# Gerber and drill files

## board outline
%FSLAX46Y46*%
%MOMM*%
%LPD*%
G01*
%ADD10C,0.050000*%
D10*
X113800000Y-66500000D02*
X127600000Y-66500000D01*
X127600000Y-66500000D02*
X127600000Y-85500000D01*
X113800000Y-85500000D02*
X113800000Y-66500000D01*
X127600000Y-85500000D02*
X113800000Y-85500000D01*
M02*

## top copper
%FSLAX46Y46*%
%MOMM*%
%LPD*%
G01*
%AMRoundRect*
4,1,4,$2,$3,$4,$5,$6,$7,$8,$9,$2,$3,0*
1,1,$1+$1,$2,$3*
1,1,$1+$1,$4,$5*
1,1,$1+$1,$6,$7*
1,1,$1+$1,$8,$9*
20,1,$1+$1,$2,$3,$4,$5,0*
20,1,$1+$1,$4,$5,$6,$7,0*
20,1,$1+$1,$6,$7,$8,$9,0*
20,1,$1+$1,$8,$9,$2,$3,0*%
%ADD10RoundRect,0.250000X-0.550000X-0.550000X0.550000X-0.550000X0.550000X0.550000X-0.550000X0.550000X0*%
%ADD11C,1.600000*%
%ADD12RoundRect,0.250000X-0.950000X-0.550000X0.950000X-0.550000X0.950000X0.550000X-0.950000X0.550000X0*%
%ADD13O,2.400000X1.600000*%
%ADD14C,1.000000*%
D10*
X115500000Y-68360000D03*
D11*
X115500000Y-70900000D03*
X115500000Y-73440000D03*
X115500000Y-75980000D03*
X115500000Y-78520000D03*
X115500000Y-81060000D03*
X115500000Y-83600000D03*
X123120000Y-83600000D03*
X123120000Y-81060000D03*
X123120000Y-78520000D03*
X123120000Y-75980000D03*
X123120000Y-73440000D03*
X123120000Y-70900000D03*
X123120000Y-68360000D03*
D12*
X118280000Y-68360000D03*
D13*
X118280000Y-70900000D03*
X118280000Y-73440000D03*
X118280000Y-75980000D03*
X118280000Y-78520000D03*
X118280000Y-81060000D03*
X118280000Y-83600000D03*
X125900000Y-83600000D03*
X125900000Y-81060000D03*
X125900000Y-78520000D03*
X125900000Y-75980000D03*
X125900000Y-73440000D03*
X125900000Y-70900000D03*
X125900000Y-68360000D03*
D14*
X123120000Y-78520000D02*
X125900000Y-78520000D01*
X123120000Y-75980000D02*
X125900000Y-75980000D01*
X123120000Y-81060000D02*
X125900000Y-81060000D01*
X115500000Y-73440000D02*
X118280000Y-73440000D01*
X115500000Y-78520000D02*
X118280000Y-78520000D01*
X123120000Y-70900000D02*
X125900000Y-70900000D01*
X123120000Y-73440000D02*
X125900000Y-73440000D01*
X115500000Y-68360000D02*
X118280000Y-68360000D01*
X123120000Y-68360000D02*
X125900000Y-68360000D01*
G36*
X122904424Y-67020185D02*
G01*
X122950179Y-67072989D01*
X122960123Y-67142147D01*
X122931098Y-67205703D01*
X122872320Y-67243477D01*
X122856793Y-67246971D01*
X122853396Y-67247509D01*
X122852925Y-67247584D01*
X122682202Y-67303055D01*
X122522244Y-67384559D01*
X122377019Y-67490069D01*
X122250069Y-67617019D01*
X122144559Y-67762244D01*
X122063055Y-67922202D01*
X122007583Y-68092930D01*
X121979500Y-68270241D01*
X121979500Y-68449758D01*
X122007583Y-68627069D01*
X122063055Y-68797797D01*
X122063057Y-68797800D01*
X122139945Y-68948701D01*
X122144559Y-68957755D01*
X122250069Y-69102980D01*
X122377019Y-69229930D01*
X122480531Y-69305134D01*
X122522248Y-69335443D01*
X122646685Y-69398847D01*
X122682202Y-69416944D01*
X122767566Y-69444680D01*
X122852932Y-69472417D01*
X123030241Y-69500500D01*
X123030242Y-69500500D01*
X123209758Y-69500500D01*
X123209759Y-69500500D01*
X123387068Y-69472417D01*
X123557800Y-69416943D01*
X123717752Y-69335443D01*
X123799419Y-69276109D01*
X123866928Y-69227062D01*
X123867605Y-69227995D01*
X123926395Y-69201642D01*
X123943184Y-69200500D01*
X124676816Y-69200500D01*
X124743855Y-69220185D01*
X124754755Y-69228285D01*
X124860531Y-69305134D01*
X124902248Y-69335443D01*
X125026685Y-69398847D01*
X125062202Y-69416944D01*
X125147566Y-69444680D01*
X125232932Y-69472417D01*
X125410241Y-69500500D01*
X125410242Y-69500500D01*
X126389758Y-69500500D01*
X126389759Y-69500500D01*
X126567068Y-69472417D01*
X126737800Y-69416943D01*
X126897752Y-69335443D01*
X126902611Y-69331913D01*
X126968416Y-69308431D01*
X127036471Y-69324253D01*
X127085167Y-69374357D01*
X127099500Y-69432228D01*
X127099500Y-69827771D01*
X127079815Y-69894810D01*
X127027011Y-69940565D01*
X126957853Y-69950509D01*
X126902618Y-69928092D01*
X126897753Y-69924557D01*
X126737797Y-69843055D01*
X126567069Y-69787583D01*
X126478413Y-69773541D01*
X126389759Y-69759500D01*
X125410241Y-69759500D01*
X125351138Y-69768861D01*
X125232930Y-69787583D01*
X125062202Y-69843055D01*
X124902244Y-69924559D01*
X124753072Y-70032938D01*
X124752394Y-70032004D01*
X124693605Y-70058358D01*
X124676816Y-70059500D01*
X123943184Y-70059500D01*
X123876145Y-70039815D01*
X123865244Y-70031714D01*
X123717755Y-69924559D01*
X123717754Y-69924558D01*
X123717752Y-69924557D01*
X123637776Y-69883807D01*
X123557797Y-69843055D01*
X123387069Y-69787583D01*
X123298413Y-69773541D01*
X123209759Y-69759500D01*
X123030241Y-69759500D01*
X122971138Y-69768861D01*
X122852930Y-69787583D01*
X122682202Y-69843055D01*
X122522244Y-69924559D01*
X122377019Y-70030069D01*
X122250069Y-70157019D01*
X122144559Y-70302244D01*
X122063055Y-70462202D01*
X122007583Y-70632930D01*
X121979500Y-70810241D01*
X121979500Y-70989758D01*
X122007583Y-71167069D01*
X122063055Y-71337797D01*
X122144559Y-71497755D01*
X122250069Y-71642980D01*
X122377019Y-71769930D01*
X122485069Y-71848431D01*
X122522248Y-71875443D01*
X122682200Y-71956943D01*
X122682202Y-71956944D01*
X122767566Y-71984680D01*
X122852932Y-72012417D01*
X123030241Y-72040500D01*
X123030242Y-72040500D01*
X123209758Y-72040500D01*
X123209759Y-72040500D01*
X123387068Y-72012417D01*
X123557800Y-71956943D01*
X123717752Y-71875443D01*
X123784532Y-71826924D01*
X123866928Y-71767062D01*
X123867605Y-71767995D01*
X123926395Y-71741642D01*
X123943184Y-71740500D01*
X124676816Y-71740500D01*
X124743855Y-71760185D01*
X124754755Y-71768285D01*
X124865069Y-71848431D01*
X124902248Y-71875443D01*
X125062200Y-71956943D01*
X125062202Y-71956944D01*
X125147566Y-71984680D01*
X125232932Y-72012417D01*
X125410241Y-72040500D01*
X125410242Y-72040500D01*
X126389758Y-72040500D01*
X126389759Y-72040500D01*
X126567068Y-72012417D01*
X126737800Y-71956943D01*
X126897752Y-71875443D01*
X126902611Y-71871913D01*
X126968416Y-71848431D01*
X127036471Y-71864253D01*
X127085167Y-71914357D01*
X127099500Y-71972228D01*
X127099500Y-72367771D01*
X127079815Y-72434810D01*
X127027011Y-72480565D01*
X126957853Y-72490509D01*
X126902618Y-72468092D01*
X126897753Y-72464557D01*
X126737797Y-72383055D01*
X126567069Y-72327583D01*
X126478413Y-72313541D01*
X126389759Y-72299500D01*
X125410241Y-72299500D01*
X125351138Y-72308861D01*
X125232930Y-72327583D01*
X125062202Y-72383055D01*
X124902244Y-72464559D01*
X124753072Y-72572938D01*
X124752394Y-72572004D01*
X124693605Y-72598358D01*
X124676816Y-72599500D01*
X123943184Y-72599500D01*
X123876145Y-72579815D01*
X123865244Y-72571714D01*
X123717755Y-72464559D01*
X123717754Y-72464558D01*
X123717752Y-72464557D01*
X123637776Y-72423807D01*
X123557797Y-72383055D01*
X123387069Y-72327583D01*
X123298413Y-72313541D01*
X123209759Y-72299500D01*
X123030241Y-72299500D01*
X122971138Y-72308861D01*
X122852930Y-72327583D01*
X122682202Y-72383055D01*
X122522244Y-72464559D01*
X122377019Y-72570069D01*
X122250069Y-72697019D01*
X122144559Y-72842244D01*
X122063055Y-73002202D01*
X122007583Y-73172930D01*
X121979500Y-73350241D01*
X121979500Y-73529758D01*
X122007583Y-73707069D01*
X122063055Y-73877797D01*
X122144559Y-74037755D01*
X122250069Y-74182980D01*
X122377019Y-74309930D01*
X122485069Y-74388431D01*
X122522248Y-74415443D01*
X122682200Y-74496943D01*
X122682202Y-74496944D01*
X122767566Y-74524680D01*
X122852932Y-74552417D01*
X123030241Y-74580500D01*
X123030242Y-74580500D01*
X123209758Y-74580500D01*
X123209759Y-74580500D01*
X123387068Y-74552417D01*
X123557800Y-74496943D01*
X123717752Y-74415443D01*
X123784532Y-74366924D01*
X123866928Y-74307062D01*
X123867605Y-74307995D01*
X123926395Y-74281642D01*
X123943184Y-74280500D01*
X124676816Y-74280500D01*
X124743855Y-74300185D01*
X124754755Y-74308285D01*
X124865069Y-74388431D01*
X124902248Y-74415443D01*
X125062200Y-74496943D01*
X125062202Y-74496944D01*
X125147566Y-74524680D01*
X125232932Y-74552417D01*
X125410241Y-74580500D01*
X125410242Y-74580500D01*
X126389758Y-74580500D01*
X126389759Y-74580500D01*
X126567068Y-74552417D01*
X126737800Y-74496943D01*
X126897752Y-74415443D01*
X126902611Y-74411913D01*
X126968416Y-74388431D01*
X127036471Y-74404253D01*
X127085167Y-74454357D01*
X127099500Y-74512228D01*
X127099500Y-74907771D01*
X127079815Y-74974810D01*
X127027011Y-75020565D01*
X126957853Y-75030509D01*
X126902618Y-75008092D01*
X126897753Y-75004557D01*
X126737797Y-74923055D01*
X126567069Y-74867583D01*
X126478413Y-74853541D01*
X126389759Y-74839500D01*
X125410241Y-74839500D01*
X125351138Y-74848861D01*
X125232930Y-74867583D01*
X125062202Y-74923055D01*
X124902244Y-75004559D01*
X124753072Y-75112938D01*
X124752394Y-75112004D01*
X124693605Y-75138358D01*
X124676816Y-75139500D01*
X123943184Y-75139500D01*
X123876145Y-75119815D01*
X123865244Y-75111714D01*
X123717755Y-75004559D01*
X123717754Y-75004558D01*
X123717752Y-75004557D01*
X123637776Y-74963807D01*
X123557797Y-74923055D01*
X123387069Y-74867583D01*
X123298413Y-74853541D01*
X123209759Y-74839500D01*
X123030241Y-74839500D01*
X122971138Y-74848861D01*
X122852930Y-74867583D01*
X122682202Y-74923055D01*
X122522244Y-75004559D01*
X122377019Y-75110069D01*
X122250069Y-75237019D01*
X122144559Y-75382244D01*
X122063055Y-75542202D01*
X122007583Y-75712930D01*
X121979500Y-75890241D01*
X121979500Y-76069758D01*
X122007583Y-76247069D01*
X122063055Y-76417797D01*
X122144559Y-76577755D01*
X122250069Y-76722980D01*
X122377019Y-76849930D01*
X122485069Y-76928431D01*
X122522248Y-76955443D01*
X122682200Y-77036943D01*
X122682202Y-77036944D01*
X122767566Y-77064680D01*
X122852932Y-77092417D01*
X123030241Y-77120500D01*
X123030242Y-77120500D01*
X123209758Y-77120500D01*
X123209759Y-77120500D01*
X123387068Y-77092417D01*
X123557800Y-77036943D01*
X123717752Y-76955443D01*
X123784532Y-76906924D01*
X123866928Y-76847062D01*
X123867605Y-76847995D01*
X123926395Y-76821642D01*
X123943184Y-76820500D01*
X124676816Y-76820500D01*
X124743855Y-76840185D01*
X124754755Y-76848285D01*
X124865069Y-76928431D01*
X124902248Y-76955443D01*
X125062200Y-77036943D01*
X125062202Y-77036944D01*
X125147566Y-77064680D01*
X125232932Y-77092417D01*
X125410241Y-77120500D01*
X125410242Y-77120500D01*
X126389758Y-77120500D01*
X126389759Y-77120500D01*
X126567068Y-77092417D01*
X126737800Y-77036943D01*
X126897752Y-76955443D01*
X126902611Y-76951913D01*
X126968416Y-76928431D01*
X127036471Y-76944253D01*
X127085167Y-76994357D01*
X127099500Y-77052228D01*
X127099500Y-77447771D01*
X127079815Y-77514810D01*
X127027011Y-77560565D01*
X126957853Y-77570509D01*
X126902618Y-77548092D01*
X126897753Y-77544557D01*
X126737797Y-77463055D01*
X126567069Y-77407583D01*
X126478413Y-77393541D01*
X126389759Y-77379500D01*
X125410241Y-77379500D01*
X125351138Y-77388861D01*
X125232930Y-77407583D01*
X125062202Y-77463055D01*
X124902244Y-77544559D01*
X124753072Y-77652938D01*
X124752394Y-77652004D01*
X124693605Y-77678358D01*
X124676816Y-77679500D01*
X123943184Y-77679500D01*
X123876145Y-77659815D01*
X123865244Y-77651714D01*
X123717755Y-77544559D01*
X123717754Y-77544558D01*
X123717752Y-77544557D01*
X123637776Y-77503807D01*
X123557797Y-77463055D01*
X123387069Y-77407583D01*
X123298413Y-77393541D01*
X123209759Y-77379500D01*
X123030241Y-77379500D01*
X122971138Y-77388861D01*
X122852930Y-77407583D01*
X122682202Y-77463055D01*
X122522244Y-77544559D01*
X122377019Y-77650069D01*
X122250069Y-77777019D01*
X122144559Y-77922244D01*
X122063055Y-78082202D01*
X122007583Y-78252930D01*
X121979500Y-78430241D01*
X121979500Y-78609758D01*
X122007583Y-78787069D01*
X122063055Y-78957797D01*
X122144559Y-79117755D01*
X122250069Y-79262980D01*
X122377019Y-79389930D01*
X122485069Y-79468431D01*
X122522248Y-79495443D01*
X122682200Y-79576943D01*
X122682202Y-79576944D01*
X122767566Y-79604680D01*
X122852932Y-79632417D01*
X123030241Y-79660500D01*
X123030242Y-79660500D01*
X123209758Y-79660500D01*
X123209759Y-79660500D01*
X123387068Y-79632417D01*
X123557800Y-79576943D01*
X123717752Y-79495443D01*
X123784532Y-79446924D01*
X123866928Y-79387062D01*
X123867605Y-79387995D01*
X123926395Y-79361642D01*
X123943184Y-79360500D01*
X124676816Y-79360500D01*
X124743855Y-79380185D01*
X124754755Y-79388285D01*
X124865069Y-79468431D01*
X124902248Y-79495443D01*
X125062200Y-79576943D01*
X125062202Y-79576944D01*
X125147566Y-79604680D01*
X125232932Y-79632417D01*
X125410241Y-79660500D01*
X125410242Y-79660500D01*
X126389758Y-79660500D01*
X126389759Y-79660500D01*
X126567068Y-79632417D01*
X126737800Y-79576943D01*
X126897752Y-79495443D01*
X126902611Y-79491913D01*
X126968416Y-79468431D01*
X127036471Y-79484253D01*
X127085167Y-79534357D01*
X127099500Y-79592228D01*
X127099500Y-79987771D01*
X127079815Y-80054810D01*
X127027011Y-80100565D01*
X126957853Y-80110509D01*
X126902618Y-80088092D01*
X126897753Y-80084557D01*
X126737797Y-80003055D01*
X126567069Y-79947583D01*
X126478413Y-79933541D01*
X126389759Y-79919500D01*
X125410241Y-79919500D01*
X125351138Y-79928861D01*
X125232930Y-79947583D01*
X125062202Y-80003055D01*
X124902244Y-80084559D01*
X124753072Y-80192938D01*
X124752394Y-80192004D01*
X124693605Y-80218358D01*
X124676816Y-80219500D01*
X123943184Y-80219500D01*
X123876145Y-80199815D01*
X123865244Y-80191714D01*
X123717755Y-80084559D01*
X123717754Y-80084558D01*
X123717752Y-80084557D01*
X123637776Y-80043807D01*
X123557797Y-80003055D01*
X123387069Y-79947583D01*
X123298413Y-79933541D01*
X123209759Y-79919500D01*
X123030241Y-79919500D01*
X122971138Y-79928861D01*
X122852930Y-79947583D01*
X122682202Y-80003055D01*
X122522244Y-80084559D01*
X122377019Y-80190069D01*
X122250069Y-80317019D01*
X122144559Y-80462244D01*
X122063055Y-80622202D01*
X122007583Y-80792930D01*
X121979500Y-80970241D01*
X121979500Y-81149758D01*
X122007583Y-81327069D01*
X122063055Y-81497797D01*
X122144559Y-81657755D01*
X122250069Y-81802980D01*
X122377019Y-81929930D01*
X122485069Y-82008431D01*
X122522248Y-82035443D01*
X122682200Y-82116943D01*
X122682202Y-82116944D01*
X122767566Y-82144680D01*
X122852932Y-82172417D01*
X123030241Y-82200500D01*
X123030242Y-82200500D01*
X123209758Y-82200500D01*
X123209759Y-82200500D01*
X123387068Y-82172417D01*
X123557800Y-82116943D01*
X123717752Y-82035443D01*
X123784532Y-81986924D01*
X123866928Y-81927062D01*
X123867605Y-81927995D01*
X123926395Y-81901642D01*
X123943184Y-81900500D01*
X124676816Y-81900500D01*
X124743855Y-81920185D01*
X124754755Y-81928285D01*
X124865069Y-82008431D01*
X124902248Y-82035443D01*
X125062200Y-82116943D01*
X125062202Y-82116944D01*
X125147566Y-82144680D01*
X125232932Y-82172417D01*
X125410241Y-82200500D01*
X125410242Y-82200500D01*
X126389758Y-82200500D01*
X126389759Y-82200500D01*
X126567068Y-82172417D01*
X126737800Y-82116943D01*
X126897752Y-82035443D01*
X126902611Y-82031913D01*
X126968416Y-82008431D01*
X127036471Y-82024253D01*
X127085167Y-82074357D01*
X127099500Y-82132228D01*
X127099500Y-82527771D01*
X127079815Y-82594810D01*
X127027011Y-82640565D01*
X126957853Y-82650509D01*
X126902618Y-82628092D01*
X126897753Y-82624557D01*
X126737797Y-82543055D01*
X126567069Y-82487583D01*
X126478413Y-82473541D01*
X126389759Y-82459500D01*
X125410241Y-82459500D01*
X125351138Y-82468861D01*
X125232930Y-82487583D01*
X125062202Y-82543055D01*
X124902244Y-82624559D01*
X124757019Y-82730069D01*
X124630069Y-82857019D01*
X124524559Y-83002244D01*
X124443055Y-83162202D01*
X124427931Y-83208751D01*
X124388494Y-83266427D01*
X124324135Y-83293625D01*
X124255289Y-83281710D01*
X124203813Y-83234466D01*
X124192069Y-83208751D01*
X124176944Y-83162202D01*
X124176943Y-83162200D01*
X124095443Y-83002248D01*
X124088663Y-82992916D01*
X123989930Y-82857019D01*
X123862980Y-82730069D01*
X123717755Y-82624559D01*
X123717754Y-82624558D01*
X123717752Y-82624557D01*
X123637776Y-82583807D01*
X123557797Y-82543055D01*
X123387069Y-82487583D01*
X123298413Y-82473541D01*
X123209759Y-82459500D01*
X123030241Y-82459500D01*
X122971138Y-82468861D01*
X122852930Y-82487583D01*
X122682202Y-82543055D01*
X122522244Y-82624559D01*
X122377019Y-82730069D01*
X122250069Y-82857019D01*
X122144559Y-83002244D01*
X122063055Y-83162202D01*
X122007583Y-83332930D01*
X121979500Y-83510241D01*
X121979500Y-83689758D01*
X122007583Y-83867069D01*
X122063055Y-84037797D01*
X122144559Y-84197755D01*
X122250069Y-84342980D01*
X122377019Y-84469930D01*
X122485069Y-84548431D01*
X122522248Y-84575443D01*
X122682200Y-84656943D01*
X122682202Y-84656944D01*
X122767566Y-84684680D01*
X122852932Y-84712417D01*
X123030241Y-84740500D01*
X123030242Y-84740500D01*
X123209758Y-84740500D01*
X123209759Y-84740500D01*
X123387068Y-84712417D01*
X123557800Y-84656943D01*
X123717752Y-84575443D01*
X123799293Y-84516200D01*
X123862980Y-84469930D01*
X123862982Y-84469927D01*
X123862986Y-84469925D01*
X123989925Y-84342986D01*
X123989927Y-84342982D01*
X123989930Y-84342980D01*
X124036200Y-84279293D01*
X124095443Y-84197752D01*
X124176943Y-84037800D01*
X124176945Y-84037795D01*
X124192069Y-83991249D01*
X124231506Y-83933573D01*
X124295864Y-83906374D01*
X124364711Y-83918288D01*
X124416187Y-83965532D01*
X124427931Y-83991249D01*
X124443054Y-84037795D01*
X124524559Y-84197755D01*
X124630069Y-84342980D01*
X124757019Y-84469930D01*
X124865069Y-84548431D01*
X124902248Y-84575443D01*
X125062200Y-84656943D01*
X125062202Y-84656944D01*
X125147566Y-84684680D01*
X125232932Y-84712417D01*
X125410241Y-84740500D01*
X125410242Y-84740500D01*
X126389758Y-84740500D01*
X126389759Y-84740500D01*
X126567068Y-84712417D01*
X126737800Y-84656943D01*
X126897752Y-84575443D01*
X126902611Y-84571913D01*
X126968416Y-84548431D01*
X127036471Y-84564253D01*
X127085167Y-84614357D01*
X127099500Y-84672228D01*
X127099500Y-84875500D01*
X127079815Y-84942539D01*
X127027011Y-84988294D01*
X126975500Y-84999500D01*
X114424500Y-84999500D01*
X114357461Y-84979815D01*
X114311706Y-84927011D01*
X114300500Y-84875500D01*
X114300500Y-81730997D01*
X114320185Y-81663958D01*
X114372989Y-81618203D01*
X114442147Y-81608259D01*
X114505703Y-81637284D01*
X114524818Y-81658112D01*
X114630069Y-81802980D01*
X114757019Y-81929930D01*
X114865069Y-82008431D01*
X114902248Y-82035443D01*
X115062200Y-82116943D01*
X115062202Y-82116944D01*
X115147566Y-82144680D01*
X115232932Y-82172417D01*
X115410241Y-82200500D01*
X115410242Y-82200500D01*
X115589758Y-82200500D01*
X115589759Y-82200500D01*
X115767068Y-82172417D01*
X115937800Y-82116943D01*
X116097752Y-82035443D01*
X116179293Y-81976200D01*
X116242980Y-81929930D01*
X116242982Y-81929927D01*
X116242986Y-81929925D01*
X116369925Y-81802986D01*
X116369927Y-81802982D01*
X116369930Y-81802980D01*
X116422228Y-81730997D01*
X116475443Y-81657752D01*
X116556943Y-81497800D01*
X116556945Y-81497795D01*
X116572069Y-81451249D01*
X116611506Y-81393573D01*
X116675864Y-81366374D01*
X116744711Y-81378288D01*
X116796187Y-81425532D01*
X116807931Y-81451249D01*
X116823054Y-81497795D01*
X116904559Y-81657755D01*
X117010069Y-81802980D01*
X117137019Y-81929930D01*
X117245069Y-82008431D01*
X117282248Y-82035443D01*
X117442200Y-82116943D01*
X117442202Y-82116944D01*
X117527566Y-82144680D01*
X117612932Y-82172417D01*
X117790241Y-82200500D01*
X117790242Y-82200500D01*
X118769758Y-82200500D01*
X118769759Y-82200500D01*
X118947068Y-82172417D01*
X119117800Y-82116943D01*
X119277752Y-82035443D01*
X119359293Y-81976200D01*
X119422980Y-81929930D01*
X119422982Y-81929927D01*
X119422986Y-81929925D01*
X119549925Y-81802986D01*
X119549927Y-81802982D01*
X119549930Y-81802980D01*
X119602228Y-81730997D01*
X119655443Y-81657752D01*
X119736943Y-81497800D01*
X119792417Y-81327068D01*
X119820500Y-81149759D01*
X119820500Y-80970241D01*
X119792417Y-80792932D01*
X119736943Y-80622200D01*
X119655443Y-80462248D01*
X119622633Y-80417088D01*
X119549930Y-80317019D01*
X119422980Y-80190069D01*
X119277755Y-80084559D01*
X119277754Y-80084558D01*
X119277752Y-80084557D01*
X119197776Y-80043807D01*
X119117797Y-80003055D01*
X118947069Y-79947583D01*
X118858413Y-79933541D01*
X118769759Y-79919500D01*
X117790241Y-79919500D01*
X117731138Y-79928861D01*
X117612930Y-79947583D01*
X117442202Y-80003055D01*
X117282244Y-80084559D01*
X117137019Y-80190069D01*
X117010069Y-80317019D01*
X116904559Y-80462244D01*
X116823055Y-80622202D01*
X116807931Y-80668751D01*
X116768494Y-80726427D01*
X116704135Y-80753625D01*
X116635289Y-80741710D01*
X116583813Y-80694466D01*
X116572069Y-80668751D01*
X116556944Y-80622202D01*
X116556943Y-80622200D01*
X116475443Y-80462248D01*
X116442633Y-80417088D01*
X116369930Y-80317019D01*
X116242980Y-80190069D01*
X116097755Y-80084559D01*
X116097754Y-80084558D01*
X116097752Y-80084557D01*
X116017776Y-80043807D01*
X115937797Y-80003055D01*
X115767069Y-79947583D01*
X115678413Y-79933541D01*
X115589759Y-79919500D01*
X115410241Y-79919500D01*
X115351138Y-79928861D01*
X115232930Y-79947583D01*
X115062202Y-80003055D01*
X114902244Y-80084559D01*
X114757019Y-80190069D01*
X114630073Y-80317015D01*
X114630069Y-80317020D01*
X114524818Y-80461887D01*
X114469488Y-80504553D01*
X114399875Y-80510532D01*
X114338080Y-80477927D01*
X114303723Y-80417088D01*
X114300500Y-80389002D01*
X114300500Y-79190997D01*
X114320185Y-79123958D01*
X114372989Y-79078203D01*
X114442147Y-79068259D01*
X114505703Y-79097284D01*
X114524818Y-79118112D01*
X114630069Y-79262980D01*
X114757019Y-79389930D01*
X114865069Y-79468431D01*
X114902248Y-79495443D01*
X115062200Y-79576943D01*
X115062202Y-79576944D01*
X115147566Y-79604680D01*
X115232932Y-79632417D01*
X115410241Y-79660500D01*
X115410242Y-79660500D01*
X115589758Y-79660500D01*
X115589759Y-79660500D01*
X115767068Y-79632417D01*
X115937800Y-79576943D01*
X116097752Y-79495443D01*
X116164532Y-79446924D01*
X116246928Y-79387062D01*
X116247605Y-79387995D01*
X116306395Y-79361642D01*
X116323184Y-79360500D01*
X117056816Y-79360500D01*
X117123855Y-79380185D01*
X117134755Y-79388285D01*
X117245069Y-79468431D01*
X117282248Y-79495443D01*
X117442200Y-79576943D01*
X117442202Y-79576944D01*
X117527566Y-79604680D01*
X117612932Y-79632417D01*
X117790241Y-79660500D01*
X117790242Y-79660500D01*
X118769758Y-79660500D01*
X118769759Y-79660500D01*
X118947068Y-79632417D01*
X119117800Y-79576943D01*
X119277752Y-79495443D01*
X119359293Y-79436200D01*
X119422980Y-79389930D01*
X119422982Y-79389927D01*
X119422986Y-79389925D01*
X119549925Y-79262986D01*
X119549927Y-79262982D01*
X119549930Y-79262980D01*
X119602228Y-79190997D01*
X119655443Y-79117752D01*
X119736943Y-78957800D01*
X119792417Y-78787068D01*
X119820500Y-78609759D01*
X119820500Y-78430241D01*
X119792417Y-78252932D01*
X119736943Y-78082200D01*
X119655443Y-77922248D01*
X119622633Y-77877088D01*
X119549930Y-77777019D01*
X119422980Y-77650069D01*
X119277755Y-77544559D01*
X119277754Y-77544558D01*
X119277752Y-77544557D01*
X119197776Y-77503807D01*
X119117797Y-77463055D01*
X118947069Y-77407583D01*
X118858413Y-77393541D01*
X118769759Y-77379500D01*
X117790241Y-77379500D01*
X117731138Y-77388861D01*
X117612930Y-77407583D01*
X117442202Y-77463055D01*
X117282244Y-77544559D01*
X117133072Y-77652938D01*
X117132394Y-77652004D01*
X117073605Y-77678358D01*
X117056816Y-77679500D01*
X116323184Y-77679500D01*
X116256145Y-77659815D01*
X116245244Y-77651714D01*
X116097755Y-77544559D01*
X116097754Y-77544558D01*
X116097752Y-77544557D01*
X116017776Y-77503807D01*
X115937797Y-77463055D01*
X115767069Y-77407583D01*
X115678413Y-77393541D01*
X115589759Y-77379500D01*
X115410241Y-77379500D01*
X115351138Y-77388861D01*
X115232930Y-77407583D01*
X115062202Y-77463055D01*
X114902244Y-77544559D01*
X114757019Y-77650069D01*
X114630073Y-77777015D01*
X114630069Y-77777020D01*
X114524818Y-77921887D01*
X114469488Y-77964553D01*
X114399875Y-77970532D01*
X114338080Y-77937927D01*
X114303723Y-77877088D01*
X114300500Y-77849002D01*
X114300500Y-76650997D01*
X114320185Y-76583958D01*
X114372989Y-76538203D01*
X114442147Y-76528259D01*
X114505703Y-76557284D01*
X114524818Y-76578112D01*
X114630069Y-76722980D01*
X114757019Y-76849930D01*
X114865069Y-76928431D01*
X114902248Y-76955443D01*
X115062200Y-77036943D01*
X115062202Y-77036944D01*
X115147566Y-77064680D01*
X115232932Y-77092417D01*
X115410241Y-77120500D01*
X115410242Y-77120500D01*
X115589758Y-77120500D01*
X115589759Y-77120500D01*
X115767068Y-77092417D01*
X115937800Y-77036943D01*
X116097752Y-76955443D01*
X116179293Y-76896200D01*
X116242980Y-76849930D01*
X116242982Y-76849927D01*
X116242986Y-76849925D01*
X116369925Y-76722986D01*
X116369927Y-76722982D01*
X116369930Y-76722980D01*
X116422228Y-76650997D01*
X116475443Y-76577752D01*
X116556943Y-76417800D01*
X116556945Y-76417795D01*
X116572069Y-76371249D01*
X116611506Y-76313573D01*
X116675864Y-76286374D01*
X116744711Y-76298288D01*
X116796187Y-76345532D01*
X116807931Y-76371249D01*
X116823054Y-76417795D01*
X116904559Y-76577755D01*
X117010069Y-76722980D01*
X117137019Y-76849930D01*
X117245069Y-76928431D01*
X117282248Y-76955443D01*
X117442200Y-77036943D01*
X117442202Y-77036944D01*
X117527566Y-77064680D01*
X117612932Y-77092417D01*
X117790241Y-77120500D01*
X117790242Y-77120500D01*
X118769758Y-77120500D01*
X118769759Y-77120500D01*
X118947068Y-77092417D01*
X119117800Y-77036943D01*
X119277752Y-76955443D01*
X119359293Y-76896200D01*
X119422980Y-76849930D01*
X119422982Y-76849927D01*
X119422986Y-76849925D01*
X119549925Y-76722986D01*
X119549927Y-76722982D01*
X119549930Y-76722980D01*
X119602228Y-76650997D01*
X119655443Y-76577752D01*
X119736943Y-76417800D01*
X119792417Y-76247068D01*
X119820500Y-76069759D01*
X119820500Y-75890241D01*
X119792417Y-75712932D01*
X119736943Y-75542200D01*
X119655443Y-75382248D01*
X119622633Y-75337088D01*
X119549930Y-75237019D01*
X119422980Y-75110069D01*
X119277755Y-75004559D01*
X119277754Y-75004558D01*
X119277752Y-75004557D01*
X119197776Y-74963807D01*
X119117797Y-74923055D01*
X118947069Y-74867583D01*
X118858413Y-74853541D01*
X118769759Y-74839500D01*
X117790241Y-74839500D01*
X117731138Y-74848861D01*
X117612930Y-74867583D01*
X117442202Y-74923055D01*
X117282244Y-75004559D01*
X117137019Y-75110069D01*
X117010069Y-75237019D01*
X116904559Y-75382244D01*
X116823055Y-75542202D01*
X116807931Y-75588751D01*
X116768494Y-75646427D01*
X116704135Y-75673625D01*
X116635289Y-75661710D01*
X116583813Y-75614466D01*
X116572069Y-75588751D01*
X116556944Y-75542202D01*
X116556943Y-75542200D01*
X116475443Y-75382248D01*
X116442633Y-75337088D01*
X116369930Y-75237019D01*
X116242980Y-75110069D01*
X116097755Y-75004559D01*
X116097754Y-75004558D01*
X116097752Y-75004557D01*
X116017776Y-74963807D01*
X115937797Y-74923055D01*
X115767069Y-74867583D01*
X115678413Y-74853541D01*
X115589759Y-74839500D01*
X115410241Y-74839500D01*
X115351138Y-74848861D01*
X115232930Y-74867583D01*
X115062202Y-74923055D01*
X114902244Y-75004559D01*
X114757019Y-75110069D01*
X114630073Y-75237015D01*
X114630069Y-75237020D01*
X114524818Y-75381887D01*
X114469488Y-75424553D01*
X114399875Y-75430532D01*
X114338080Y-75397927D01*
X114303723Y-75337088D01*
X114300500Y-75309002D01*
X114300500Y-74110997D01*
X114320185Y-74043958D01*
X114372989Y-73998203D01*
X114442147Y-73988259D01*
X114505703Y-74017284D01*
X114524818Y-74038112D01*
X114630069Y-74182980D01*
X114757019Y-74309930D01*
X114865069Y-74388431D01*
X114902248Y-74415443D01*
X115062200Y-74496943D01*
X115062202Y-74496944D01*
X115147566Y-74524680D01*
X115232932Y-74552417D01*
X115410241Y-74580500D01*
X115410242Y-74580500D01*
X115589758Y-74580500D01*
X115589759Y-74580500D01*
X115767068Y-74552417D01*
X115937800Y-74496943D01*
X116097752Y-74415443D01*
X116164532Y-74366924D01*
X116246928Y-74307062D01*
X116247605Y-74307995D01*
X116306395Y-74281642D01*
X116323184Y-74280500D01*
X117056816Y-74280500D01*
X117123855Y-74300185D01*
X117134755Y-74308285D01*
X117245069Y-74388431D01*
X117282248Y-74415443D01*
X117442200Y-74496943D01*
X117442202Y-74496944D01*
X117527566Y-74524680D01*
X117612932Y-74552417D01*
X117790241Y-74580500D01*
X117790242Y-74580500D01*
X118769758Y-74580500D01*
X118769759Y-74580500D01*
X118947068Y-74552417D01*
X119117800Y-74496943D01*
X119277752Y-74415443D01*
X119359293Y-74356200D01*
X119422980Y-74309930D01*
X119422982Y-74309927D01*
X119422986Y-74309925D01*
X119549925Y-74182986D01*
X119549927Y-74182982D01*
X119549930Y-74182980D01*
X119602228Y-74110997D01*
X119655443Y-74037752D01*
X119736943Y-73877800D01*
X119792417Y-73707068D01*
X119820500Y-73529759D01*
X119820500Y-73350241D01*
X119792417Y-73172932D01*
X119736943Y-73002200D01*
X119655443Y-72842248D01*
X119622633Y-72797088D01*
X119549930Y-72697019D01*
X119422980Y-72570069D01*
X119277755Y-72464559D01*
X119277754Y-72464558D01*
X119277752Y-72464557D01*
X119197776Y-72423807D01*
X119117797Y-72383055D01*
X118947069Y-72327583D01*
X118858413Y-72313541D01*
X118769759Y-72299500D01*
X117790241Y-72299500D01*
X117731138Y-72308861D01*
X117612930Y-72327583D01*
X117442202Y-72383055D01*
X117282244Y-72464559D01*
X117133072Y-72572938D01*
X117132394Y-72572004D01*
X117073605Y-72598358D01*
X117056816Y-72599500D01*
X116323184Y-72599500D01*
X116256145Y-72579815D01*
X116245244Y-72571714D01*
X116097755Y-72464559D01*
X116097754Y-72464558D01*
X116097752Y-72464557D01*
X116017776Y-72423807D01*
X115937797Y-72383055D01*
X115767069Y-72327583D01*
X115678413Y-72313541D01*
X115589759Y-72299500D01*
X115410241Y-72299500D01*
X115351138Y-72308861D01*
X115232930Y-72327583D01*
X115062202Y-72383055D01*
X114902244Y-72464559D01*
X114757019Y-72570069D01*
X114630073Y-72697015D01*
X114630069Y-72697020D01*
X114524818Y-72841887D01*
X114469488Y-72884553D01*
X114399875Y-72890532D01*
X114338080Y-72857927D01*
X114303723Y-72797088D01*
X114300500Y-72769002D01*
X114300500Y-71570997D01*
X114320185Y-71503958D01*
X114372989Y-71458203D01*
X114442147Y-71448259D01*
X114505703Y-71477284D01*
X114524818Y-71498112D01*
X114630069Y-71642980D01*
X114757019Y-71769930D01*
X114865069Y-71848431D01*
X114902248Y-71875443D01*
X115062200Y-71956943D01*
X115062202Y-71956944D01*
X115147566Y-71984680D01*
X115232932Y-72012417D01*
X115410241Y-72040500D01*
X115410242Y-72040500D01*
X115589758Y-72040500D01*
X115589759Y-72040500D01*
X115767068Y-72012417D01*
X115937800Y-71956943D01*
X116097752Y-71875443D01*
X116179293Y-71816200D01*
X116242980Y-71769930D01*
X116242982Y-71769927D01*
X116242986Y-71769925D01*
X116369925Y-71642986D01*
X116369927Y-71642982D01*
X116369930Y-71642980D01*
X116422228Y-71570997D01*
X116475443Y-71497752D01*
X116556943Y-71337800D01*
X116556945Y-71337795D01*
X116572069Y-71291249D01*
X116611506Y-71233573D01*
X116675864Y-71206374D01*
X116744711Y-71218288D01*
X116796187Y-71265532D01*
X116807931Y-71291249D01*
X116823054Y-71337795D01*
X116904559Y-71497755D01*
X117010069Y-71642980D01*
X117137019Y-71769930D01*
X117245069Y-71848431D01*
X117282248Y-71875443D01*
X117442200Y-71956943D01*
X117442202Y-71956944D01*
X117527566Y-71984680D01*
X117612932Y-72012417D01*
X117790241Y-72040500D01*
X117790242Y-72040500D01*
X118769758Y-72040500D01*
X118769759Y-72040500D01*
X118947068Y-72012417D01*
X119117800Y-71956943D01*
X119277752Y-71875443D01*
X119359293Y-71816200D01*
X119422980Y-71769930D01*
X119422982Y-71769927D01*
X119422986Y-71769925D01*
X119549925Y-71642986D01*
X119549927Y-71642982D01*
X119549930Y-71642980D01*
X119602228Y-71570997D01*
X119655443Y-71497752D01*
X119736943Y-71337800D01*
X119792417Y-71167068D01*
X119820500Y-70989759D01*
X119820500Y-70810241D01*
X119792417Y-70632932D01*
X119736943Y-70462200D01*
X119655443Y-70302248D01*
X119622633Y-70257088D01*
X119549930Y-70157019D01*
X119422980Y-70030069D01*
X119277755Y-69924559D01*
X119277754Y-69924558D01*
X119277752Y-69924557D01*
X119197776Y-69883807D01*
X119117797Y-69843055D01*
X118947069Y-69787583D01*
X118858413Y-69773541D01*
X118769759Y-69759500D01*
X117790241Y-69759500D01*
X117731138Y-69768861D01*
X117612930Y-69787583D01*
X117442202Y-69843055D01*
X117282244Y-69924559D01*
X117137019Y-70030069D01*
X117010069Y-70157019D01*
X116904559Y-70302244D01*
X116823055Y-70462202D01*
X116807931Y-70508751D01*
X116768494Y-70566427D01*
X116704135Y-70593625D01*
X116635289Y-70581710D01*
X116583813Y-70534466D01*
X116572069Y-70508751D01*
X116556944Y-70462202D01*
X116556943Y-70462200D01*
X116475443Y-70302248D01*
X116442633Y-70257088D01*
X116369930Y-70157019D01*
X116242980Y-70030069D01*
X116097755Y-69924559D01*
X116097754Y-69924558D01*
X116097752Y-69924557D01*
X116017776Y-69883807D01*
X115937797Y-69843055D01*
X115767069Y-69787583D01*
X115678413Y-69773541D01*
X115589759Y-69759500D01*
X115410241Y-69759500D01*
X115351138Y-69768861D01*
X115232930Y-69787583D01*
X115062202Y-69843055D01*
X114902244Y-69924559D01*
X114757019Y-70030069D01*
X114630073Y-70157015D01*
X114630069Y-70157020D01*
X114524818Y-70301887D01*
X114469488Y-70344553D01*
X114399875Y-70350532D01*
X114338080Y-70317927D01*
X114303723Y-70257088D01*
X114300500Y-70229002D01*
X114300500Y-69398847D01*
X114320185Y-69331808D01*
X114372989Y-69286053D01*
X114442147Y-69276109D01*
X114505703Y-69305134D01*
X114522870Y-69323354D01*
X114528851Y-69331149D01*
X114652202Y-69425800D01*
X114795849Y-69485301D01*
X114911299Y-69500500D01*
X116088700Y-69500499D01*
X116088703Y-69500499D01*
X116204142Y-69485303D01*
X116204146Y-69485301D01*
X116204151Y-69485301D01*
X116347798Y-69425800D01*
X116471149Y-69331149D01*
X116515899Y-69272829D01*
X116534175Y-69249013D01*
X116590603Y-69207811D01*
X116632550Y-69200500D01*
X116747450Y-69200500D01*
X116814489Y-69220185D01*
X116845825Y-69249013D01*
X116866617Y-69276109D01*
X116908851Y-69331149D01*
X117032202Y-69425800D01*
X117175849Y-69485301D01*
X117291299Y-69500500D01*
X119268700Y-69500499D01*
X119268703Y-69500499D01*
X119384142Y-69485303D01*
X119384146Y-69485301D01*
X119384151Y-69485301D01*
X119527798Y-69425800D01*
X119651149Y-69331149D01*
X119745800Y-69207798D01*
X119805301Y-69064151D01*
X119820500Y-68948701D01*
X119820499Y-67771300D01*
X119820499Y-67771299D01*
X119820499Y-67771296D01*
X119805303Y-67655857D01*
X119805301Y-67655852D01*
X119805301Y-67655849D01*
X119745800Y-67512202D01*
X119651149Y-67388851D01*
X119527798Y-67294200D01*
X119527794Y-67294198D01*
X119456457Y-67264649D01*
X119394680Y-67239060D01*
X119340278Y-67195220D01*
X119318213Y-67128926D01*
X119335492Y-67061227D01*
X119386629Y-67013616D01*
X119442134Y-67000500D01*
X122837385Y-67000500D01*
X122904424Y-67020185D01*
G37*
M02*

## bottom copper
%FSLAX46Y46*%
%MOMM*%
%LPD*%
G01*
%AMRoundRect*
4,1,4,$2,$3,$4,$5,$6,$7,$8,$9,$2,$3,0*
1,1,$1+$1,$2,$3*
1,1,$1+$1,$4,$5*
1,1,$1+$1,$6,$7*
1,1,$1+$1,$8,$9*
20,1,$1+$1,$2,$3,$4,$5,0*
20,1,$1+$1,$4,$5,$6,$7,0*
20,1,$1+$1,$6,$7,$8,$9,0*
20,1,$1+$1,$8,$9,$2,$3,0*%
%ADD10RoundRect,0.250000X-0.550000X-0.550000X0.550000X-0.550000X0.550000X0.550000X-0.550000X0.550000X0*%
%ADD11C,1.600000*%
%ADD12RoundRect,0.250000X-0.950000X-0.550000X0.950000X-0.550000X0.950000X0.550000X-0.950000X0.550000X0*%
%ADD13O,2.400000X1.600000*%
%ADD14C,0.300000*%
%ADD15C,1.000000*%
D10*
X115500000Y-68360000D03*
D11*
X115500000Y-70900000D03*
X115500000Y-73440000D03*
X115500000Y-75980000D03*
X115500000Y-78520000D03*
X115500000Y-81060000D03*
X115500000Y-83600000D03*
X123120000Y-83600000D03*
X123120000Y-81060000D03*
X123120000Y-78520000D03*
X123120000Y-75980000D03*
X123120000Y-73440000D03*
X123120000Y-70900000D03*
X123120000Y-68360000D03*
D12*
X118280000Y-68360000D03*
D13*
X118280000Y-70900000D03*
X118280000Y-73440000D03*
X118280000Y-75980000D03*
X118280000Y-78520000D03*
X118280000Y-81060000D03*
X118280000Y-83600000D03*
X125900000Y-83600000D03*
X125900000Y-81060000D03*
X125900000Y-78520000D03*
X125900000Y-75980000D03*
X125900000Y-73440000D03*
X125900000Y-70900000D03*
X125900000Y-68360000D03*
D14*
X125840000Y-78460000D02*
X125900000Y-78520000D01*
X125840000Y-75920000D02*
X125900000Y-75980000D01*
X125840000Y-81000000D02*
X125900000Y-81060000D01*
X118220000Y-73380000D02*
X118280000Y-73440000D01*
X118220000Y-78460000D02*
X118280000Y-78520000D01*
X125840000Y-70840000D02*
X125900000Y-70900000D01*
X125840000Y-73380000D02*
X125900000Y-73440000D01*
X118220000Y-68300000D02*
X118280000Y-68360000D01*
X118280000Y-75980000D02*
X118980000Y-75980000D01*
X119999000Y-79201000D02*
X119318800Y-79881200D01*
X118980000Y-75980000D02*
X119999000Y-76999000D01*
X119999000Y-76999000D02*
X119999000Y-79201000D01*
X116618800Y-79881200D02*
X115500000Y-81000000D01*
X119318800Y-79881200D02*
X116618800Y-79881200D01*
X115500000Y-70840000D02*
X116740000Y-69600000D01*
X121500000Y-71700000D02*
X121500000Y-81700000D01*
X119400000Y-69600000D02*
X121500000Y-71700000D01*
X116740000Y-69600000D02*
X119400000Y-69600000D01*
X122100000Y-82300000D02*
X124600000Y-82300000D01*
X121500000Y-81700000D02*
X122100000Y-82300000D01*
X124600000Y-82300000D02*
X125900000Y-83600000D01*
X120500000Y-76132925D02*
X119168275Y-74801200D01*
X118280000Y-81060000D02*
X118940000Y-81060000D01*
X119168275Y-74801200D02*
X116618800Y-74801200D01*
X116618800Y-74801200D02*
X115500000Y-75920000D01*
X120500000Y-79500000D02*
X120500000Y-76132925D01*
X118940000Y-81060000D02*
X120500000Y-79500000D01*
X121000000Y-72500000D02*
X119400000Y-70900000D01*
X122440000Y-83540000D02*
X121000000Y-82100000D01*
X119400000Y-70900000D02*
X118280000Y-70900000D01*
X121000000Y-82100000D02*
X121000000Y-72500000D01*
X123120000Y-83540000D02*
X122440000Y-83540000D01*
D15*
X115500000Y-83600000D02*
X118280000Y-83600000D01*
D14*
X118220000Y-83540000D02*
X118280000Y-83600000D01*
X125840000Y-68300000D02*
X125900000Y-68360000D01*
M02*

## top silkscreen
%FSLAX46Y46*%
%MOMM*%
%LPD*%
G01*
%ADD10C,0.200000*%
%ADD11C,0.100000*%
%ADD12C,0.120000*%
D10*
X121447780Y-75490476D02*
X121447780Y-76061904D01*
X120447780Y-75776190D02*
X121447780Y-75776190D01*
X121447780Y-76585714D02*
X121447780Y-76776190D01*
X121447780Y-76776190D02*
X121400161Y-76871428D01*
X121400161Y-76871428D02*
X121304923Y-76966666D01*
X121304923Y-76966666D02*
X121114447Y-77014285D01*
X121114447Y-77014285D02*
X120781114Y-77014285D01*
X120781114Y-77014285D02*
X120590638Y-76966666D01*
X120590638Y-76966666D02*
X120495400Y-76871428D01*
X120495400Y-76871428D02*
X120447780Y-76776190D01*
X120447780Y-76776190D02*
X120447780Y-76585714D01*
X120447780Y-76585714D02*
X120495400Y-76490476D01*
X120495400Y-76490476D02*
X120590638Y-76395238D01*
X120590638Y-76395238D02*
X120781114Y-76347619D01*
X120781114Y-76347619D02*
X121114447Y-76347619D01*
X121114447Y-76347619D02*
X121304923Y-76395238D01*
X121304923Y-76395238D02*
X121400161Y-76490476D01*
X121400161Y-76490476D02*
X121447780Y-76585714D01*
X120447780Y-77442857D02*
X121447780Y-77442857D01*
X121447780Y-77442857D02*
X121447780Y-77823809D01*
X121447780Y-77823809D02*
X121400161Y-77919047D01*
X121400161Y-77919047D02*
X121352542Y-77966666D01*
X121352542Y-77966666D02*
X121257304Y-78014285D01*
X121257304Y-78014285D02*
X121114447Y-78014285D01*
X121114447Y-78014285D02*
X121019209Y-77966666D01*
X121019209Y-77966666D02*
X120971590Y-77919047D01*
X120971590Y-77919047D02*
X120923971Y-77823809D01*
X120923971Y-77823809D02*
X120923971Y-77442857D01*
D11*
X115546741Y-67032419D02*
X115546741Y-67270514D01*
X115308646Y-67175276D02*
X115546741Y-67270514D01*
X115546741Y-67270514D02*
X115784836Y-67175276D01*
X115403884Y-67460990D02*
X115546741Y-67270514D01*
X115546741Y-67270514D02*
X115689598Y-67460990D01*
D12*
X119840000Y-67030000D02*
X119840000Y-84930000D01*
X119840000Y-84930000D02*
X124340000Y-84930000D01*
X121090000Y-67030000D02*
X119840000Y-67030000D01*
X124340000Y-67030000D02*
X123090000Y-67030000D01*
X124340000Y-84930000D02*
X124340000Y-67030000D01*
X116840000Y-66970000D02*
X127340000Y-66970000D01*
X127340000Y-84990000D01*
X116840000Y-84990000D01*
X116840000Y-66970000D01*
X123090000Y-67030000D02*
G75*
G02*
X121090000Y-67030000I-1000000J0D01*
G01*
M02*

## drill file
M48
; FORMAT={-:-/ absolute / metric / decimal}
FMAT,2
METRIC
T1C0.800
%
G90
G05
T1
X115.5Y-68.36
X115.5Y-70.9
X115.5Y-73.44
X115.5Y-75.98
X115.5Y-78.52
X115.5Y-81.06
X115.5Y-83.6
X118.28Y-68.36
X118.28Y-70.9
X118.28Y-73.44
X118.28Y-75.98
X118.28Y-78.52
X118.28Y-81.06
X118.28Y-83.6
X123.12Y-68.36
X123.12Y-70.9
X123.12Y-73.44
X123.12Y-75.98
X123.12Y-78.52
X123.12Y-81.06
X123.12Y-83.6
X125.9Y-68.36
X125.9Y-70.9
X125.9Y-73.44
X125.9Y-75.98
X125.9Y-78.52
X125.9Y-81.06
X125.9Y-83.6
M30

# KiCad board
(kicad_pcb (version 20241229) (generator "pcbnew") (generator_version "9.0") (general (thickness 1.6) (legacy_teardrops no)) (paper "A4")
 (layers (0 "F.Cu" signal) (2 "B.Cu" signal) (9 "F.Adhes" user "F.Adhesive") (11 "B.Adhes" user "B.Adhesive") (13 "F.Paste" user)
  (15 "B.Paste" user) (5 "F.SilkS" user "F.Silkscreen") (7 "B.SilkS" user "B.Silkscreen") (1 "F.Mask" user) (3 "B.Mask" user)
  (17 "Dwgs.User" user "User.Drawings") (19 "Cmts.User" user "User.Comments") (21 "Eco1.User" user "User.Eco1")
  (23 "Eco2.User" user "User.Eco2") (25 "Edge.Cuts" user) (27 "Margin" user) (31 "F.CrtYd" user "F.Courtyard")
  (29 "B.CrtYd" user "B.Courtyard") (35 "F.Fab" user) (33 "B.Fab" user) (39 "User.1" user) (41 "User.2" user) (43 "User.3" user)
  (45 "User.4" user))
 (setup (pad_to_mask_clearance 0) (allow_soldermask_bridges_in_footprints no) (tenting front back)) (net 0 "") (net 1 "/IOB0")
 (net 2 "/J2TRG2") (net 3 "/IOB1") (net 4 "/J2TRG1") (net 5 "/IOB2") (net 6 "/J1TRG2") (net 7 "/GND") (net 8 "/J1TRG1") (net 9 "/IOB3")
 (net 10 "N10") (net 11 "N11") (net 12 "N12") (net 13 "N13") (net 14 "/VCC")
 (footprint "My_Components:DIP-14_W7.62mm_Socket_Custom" (layer "F.Cu") (at 115.5 68.36)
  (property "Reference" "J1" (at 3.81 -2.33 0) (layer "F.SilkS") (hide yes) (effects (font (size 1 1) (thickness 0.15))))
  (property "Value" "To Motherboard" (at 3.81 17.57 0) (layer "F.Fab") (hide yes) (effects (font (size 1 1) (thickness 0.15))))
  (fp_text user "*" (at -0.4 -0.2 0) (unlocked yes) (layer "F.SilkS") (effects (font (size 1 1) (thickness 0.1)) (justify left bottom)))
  (pad "1" thru_hole roundrect (at 0 0) (size 1.6 1.6) (drill 0.8) (layers "*.Cu" "*.Mask") (remove_unused_layers no)
   (roundrect_rratio 0.15625) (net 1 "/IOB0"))
  (pad "2" thru_hole circle (at 0 2.54) (size 1.6 1.6) (drill 0.8) (layers "*.Cu" "*.Mask") (remove_unused_layers no) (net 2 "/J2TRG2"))
  (pad "3" thru_hole circle (at 0 5.08) (size 1.6 1.6) (drill 0.8) (layers "*.Cu" "*.Mask") (remove_unused_layers no) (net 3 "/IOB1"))
  (pad "4" thru_hole circle (at 0 7.62) (size 1.6 1.6) (drill 0.8) (layers "*.Cu" "*.Mask") (remove_unused_layers no) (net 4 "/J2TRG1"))
  (pad "5" thru_hole circle (at 0 10.16) (size 1.6 1.6) (drill 0.8) (layers "*.Cu" "*.Mask") (remove_unused_layers no) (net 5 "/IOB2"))
  (pad "6" thru_hole circle (at 0 12.7) (size 1.6 1.6) (drill 0.8) (layers "*.Cu" "*.Mask") (remove_unused_layers no) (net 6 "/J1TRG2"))
  (pad "7" thru_hole circle (at 0 15.24) (size 1.6 1.6) (drill 0.8) (layers "*.Cu" "*.Mask") (remove_unused_layers no) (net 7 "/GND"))
  (pad "8" thru_hole circle (at 7.62 15.24) (size 1.6 1.6) (drill 0.8) (layers "*.Cu" "*.Mask") (remove_unused_layers no) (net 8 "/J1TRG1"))
  (pad "9" thru_hole circle (at 7.62 12.7) (size 1.6 1.6) (drill 0.8) (layers "*.Cu" "*.Mask") (remove_unused_layers no) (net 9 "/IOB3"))
  (pad "10" thru_hole circle (at 7.62 10.16) (size 1.6 1.6) (drill 0.8) (layers "*.Cu" "*.Mask") (remove_unused_layers no) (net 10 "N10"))
  (pad "11" thru_hole circle (at 7.62 7.62) (size 1.6 1.6) (drill 0.8) (layers "*.Cu" "*.Mask") (remove_unused_layers no) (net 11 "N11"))
  (pad "12" thru_hole circle (at 7.62 5.08) (size 1.6 1.6) (drill 0.8) (layers "*.Cu" "*.Mask") (remove_unused_layers no) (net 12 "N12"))
  (pad "13" thru_hole circle (at 7.62 2.54) (size 1.6 1.6) (drill 0.8) (layers "*.Cu" "*.Mask") (remove_unused_layers no) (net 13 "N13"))
  (pad "14" thru_hole circle (at 7.62 0) (size 1.6 1.6) (drill 0.8) (layers "*.Cu" "*.Mask") (remove_unused_layers no) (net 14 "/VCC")))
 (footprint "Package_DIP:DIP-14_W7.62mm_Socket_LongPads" (layer "F.Cu") (at 118.28 68.36)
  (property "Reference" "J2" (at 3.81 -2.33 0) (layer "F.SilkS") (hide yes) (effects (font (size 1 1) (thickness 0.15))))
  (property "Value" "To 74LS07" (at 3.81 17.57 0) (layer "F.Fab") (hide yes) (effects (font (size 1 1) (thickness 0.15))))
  (fp_line (start 1.56 -1.33) (end 1.56 16.57) (stroke (width 0.12) (type solid)) (layer "F.SilkS"))
  (fp_line (start 1.56 16.57) (end 6.06 16.57) (stroke (width 0.12) (type solid)) (layer "F.SilkS"))
  (fp_line (start 2.81 -1.33) (end 1.56 -1.33) (stroke (width 0.12) (type solid)) (layer "F.SilkS"))
  (fp_line (start 6.06 -1.33) (end 4.81 -1.33) (stroke (width 0.12) (type solid)) (layer "F.SilkS"))
  (fp_line (start 6.06 16.57) (end 6.06 -1.33) (stroke (width 0.12) (type solid)) (layer "F.SilkS"))
  (fp_rect (start -1.44 -1.39) (end 9.06 16.63) (stroke (width 0.12) (type solid)) (fill no) (layer "F.SilkS"))
  (fp_arc (start 4.81 -1.33) (mid 3.81 -0.33) (end 2.81 -1.33) (stroke (width 0.12) (type solid)) (layer "F.SilkS"))
  (pad "1" thru_hole roundrect (at 0 0) (size 2.4 1.6) (drill 0.8) (layers "*.Cu" "*.Mask") (remove_unused_layers no)
   (roundrect_rratio 0.15625) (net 1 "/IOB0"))
  (pad "2" thru_hole oval (at 0 2.54) (size 2.4 1.6) (drill 0.8) (layers "*.Cu" "*.Mask") (remove_unused_layers no) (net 8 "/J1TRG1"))
  (pad "3" thru_hole oval (at 0 5.08) (size 2.4 1.6) (drill 0.8) (layers "*.Cu" "*.Mask") (remove_unused_layers no) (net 3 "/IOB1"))
  (pad "4" thru_hole oval (at 0 7.62) (size 2.4 1.6) (drill 0.8) (layers "*.Cu" "*.Mask") (remove_unused_layers no) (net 6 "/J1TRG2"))
  (pad "5" thru_hole oval (at 0 10.16) (size 2.4 1.6) (drill 0.8) (layers "*.Cu" "*.Mask") (remove_unused_layers no) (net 5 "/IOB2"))
  (pad "6" thru_hole oval (at 0 12.7) (size 2.4 1.6) (drill 0.8) (layers "*.Cu" "*.Mask") (remove_unused_layers no) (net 4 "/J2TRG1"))
  (pad "7" thru_hole oval (at 0 15.24) (size 2.4 1.6) (drill 0.8) (layers "*.Cu" "*.Mask") (remove_unused_layers no) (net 7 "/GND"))
  (pad "8" thru_hole oval (at 7.62 15.24) (size 2.4 1.6) (drill 0.8) (layers "*.Cu" "*.Mask") (remove_unused_layers no) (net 2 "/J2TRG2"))
  (pad "9" thru_hole oval (at 7.62 12.7) (size 2.4 1.6) (drill 0.8) (layers "*.Cu" "*.Mask") (remove_unused_layers no) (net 9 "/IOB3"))
  (pad "10" thru_hole oval (at 7.62 10.16) (size 2.4 1.6) (drill 0.8) (layers "*.Cu" "*.Mask") (remove_unused_layers no) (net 10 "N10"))
  (pad "11" thru_hole oval (at 7.62 7.62) (size 2.4 1.6) (drill 0.8) (layers "*.Cu" "*.Mask") (remove_unused_layers no) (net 11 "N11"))
  (pad "12" thru_hole oval (at 7.62 5.08) (size 2.4 1.6) (drill 0.8) (layers "*.Cu" "*.Mask") (remove_unused_layers no) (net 12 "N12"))
  (pad "13" thru_hole oval (at 7.62 2.54) (size 2.4 1.6) (drill 0.8) (layers "*.Cu" "*.Mask") (remove_unused_layers no) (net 13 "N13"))
  (pad "14" thru_hole oval (at 7.62 0) (size 2.4 1.6) (drill 0.8) (layers "*.Cu" "*.Mask") (remove_unused_layers no) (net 14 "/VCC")))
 (gr_line (start 113.8 66.5) (end 127.6 66.5) (stroke (width 0.05) (type default)) (layer "Edge.Cuts"))
 (gr_line (start 127.6 66.5) (end 127.6 85.5) (stroke (width 0.05) (type default)) (layer "Edge.Cuts"))
 (gr_line (start 113.8 85.5) (end 113.8 66.5) (stroke (width 0.05) (type default)) (layer "Edge.Cuts"))
 (gr_line (start 127.6 85.5) (end 113.8 85.5) (stroke (width 0.05) (type default)) (layer "Edge.Cuts"))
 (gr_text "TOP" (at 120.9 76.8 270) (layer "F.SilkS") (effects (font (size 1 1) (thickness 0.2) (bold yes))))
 (segment (start 123.12 78.52) (end 125.9 78.52) (width 1) (layer "F.Cu") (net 10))
 (segment (start 125.84 78.46) (end 125.9 78.52) (width 0.3) (layer "B.Cu") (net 10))
 (segment (start 123.12 75.98) (end 125.9 75.98) (width 1) (layer "F.Cu") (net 11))
 (segment (start 125.84 75.92) (end 125.9 75.98) (width 0.3) (layer "B.Cu") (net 11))
 (segment (start 123.12 81.06) (end 125.9 81.06) (width 1) (layer "F.Cu") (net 9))
 (segment (start 125.84 81) (end 125.9 81.06) (width 0.3) (layer "B.Cu") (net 9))
 (segment (start 115.5 73.44) (end 118.28 73.44) (width 1) (layer "F.Cu") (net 3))
 (segment (start 118.22 73.38) (end 118.28 73.44) (width 0.3) (layer "B.Cu") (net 3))
 (segment (start 115.5 78.52) (end 118.28 78.52) (width 1) (layer "F.Cu") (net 5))
 (segment (start 118.22 78.46) (end 118.28 78.52) (width 0.3) (layer "B.Cu") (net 5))
 (segment (start 123.12 70.9) (end 125.9 70.9) (width 1) (layer "F.Cu") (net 13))
 (segment (start 125.84 70.84) (end 125.9 70.9) (width 0.3) (layer "B.Cu") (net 13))
 (segment (start 123.12 73.44) (end 125.9 73.44) (width 1) (layer "F.Cu") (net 12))
 (segment (start 125.84 73.38) (end 125.9 73.44) (width 0.3) (layer "B.Cu") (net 12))
 (segment (start 115.5 68.36) (end 118.28 68.36) (width 1) (layer "F.Cu") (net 1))
 (segment (start 118.22 68.3) (end 118.28 68.36) (width 0.3) (layer "B.Cu") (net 1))
 (segment (start 118.28 75.98) (end 118.98 75.98) (width 0.3) (layer "B.Cu") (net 6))
 (segment (start 119.999 79.201) (end 119.3188 79.8812) (width 0.3) (layer "B.Cu") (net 6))
 (segment (start 118.98 75.98) (end 119.999 76.999) (width 0.3) (layer "B.Cu") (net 6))
 (segment (start 119.999 76.999) (end 119.999 79.201) (width 0.3) (layer "B.Cu") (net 6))
 (segment (start 116.6188 79.8812) (end 115.5 81) (width 0.3) (layer "B.Cu") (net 6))
 (segment (start 119.3188 79.8812) (end 116.6188 79.8812) (width 0.3) (layer "B.Cu") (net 6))
 (segment (start 115.5 70.84) (end 116.74 69.6) (width 0.3) (layer "B.Cu") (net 2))
 (segment (start 121.5 71.7) (end 121.5 81.7) (width 0.3) (layer "B.Cu") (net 2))
 (segment (start 119.4 69.6) (end 121.5 71.7) (width 0.3) (layer "B.Cu") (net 2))
 (segment (start 116.74 69.6) (end 119.4 69.6) (width 0.3) (layer "B.Cu") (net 2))
 (segment (start 122.1 82.3) (end 124.6 82.3) (width 0.3) (layer "B.Cu") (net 2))
 (segment (start 121.5 81.7) (end 122.1 82.3) (width 0.3) (layer "B.Cu") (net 2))
 (segment (start 124.6 82.3) (end 125.9 83.6) (width 0.3) (layer "B.Cu") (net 2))
 (segment (start 120.5 76.132925) (end 119.168275 74.8012) (width 0.3) (layer "B.Cu") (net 4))
 (segment (start 118.28 81.06) (end 118.94 81.06) (width 0.3) (layer "B.Cu") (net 4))
 (segment (start 119.168275 74.8012) (end 116.6188 74.8012) (width 0.3) (layer "B.Cu") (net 4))
 (segment (start 116.6188 74.8012) (end 115.5 75.92) (width 0.3) (layer "B.Cu") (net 4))
 (segment (start 120.5 79.5) (end 120.5 76.132925) (width 0.3) (layer "B.Cu") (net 4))
 (segment (start 118.94 81.06) (end 120.5 79.5) (width 0.3) (layer "B.Cu") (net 4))
 (segment (start 121 72.5) (end 119.4 70.9) (width 0.3) (layer "B.Cu") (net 8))
 (segment (start 122.44 83.54) (end 121 82.1) (width 0.3) (layer "B.Cu") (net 8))
 (segment (start 119.4 70.9) (end 118.28 70.9) (width 0.3) (layer "B.Cu") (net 8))
 (segment (start 121 82.1) (end 121 72.5) (width 0.3) (layer "B.Cu") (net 8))
 (segment (start 123.12 83.54) (end 122.44 83.54) (width 0.3) (layer "B.Cu") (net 8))
 (segment (start 115.5 83.6) (end 118.28 83.6) (width 1) (layer "B.Cu") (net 7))
 (segment (start 118.22 83.54) (end 118.28 83.6) (width 0.3) (layer "B.Cu") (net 7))
 (segment (start 123.12 68.36) (end 125.9 68.36) (width 1) (layer "F.Cu") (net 14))
 (segment (start 125.84 68.3) (end 125.9 68.36) (width 0.3) (layer "B.Cu") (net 14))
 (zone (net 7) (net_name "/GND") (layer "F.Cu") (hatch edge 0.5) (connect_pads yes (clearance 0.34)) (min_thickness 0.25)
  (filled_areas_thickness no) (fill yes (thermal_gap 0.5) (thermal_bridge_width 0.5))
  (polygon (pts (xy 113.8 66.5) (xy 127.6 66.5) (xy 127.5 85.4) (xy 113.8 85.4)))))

